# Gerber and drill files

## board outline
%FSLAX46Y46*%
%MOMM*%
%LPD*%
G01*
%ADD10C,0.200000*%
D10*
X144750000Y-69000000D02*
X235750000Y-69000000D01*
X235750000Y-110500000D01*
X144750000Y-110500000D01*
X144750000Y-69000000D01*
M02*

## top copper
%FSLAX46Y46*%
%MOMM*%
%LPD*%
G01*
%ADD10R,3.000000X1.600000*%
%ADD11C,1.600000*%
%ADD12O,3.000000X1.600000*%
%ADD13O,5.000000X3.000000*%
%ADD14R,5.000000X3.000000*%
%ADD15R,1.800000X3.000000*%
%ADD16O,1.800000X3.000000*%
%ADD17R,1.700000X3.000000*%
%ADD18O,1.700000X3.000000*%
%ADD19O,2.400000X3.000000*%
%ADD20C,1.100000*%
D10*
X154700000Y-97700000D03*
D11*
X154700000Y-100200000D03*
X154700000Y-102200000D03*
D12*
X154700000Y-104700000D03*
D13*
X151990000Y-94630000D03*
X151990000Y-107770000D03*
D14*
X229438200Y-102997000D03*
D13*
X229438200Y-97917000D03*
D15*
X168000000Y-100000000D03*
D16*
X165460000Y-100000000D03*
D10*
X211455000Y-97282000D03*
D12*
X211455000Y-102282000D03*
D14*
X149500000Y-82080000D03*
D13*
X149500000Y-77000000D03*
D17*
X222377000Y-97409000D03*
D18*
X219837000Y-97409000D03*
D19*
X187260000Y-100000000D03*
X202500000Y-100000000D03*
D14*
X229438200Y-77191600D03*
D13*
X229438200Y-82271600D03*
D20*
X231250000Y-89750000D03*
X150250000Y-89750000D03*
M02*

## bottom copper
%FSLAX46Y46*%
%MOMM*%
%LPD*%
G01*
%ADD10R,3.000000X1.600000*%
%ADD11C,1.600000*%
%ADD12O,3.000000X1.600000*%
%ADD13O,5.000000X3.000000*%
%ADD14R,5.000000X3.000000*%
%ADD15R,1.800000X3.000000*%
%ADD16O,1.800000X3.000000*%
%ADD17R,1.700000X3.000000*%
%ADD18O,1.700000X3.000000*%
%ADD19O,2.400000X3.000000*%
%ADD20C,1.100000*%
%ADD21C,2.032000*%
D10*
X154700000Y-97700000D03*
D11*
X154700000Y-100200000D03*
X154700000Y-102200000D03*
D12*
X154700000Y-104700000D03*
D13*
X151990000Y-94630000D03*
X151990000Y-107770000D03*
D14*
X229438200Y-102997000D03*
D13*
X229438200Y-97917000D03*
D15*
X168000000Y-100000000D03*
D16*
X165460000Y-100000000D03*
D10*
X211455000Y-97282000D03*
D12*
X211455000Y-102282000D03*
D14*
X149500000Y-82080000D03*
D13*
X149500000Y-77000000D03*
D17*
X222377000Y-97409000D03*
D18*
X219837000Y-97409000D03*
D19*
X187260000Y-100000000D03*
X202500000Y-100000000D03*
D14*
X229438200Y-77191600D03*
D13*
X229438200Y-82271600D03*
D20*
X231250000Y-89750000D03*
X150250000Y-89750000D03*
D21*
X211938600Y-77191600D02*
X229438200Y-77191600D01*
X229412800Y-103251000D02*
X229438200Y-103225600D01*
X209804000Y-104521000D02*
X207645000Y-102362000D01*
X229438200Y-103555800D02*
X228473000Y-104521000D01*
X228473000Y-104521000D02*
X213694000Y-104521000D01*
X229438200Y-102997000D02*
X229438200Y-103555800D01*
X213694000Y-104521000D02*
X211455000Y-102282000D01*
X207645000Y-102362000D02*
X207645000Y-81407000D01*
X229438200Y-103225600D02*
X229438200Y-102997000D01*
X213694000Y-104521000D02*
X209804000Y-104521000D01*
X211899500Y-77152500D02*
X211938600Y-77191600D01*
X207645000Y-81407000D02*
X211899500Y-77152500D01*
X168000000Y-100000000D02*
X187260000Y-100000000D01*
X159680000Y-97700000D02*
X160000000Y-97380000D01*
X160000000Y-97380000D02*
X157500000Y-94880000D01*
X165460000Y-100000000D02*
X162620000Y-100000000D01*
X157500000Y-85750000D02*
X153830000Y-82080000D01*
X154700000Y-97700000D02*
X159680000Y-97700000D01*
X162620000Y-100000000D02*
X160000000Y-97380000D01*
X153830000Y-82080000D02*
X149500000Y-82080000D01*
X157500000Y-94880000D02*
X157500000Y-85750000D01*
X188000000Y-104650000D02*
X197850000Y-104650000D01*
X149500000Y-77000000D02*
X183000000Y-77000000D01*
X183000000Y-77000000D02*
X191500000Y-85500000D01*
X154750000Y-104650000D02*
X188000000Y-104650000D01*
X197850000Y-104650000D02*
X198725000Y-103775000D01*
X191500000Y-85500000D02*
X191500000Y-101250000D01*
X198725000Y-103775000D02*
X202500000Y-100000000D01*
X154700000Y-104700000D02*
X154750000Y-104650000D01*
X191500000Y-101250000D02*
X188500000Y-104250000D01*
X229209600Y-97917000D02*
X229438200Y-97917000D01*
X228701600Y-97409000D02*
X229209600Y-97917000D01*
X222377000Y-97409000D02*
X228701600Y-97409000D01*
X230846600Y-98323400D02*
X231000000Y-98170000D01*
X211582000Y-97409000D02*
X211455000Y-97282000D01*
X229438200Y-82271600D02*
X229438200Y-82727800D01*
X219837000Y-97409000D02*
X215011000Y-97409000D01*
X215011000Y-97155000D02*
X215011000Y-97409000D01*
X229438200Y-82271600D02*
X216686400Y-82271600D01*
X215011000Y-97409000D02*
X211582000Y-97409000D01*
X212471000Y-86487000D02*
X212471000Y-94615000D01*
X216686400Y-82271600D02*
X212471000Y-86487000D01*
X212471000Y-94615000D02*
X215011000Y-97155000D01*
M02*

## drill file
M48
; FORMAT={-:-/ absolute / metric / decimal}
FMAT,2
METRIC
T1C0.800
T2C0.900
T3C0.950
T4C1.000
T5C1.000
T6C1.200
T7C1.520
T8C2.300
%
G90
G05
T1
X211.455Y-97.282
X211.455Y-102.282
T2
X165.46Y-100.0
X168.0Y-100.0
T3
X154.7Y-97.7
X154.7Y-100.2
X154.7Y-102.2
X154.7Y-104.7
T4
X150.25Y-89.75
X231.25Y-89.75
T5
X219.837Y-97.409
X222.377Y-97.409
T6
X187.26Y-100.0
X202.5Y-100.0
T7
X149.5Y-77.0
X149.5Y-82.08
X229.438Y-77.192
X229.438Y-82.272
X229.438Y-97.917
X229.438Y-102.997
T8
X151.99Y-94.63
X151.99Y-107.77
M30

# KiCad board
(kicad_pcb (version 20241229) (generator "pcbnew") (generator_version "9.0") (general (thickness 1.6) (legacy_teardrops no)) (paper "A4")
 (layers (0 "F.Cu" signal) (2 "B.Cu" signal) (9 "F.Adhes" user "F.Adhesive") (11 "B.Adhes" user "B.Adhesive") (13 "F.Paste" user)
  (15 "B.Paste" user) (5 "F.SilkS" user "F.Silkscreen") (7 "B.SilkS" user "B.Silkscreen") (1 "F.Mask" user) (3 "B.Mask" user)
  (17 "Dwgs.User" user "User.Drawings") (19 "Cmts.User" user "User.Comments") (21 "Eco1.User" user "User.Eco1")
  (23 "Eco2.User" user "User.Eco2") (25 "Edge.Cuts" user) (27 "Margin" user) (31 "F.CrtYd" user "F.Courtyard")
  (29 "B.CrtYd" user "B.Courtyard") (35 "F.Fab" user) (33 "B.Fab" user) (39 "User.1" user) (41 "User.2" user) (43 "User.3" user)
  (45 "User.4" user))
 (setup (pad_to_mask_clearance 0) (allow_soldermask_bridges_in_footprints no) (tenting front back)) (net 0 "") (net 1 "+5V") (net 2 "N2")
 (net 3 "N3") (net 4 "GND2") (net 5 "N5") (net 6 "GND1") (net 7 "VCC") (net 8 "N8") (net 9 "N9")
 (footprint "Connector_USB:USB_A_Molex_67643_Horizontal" (layer "F.Cu") (at 154.7 97.7 -90)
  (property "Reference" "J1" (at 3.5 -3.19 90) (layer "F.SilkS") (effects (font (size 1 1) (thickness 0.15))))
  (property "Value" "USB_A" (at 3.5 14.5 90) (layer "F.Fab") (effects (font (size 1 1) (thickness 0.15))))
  (pad "1" thru_hole rect (at 0 0 270) (size 1.6 3) (drill 0.95) (layers "*.Cu" "*.Mask") (remove_unused_layers no) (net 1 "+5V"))
  (pad "2" thru_hole circle (at 2.5 0 270) (size 1.6 1.6) (drill 0.95) (layers "*.Cu" "*.Mask") (remove_unused_layers no) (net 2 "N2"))
  (pad "3" thru_hole circle (at 4.5 0 270) (size 1.6 1.6) (drill 0.95) (layers "*.Cu" "*.Mask") (remove_unused_layers no) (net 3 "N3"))
  (pad "4" thru_hole oval (at 7 0 270) (size 1.6 3) (drill 0.95) (layers "*.Cu" "*.Mask") (remove_unused_layers no) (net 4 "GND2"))
  (pad "5" thru_hole oval (at -3.07 2.71 270) (size 3 5) (drill 2.3) (layers "*.Cu" "*.Mask") (remove_unused_layers no) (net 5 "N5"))
  (pad "5" thru_hole oval (at 10.07 2.71 270) (size 3 5) (drill 2.3) (layers "*.Cu" "*.Mask") (remove_unused_layers no) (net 5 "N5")))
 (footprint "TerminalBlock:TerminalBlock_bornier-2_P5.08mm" (layer "F.Cu") (at 229.4382 102.997 90)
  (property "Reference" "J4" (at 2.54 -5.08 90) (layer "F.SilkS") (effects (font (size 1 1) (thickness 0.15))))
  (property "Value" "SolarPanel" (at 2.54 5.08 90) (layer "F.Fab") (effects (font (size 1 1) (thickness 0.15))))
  (pad "1" thru_hole rect (at 0 0 90) (size 3 5) (drill 1.52) (layers "*.Cu" "*.Mask") (remove_unused_layers no) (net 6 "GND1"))
  (pad "2" thru_hole oval (at 5.08 0 90) (size 3 5) (drill 1.52) (layers "*.Cu" "*.Mask") (remove_unused_layers no) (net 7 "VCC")))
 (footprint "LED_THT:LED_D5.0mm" (layer "F.Cu") (at 168 100 180)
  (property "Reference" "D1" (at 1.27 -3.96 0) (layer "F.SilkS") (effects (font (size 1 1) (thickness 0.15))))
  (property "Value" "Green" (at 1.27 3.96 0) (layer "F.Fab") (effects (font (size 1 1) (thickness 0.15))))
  (pad "1" thru_hole rect (at 0 0 180) (size 1.8 3) (drill 0.9) (layers "*.Cu" "*.Mask") (remove_unused_layers no) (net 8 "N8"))
  (pad "2" thru_hole oval (at 2.54 0 180) (size 1.8 3) (drill 0.9) (layers "*.Cu" "*.Mask") (remove_unused_layers no) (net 1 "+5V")))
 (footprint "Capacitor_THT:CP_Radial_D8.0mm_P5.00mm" (layer "F.Cu") (at 211.455 97.282 -90)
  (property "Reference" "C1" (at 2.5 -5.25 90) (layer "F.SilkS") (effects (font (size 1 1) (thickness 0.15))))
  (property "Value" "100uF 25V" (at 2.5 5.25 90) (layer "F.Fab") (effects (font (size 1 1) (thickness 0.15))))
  (pad "1" thru_hole rect (at 0 0 270) (size 1.6 3) (drill 0.8) (layers "*.Cu" "*.Mask") (remove_unused_layers no) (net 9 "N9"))
  (pad "2" thru_hole oval (at 5 0 270) (size 1.6 3) (drill 0.8) (layers "*.Cu" "*.Mask") (remove_unused_layers no) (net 6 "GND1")))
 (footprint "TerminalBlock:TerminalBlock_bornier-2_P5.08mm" (layer "F.Cu") (at 149.5 82.08 90)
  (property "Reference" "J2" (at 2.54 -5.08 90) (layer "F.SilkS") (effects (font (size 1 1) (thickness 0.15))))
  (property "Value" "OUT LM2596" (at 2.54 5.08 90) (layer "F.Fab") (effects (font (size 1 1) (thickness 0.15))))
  (pad "1" thru_hole rect (at 0 0 90) (size 3 5) (drill 1.52) (layers "*.Cu" "*.Mask") (remove_unused_layers no) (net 1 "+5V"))
  (pad "2" thru_hole oval (at 5.08 0 90) (size 3 5) (drill 1.52) (layers "*.Cu" "*.Mask") (remove_unused_layers no) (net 4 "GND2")))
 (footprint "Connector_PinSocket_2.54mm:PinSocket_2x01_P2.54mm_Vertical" (layer "F.Cu") (at 222.377 97.409)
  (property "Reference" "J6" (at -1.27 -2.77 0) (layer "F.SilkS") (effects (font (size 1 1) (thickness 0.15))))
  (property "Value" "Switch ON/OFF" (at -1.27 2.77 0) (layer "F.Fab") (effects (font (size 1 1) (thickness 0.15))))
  (pad "1" thru_hole rect (at 0 0) (size 1.7 3) (drill 1) (layers "*.Cu" "*.Mask") (remove_unused_layers no) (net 7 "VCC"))
  (pad "2" thru_hole oval (at -2.54 0) (size 1.7 3) (drill 1) (layers "*.Cu" "*.Mask") (remove_unused_layers no) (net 9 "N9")))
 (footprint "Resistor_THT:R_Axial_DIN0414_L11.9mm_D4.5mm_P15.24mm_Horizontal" (layer "F.Cu") (at 187.26 100)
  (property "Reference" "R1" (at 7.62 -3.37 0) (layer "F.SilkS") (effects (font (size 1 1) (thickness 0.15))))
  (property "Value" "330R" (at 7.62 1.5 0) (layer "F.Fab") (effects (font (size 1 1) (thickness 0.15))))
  (pad "1" thru_hole oval (at 0 0) (size 2.4 3) (drill 1.2) (layers "*.Cu" "*.Mask") (remove_unused_layers no) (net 8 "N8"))
  (pad "2" thru_hole oval (at 15.24 0) (size 2.4 3) (drill 1.2) (layers "*.Cu" "*.Mask") (remove_unused_layers no) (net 4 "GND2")))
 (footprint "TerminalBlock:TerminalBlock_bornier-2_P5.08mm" (layer "F.Cu") (at 229.4382 77.1916 -90)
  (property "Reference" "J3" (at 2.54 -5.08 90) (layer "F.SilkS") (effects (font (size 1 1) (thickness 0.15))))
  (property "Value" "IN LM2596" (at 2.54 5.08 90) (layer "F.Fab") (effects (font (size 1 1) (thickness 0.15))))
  (pad "1" thru_hole rect (at 0 0 270) (size 3 5) (drill 1.52) (layers "*.Cu" "*.Mask") (remove_unused_layers no) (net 6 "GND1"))
  (pad "2" thru_hole oval (at 5.08 0 270) (size 3 5) (drill 1.52) (layers "*.Cu" "*.Mask") (remove_unused_layers no) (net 9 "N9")))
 (gr_rect (start 144.75 69) (end 235.75 110.5) (stroke (width 0.2) (type solid)) (fill no) (layer "Edge.Cuts"))
 (via (at 231.25 89.75) (size 1.1) (drill 1) (layers "F.Cu" "B.Cu") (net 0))
 (via (at 150.25 89.75) (size 1.1) (drill 1) (layers "F.Cu" "B.Cu") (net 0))
 (segment (start 211.9386 77.1916) (end 229.4382 77.1916) (width 2.032) (layer "B.Cu") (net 6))
 (segment (start 229.4128 103.251) (end 229.4382 103.2256) (width 2.032) (layer "B.Cu") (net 6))
 (segment (start 209.804 104.521) (end 207.645 102.362) (width 2.032) (layer "B.Cu") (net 6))
 (segment (start 229.4382 103.5558) (end 228.473 104.521) (width 2.032) (layer "B.Cu") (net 6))
 (segment (start 228.473 104.521) (end 213.694 104.521) (width 2.032) (layer "B.Cu") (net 6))
 (segment (start 229.4382 102.997) (end 229.4382 103.5558) (width 2.032) (layer "B.Cu") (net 6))
 (segment (start 213.694 104.521) (end 211.455 102.282) (width 2.032) (layer "B.Cu") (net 6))
 (segment (start 207.645 102.362) (end 207.645 81.407) (width 2.032) (layer "B.Cu") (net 6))
 (segment (start 229.4382 103.2256) (end 229.4382 102.997) (width 2.032) (layer "B.Cu") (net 6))
 (segment (start 213.694 104.521) (end 209.804 104.521) (width 2.032) (layer "B.Cu") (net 6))
 (segment (start 211.8995 77.1525) (end 211.9386 77.1916) (width 2.032) (layer "B.Cu") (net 6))
 (segment (start 207.645 81.407) (end 211.8995 77.1525) (width 2.032) (layer "B.Cu") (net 6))
 (segment (start 168 100) (end 187.26 100) (width 2.032) (layer "B.Cu") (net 8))
 (segment (start 159.68 97.7) (end 160 97.38) (width 2.032) (layer "B.Cu") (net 1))
 (segment (start 160 97.38) (end 157.5 94.88) (width 2.032) (layer "B.Cu") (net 1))
 (segment (start 165.46 100) (end 162.62 100) (width 2.032) (layer "B.Cu") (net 1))
 (segment (start 157.5 85.75) (end 153.83 82.08) (width 2.032) (layer "B.Cu") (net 1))
 (segment (start 154.7 97.7) (end 159.68 97.7) (width 2.032) (layer "B.Cu") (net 1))
 (segment (start 162.62 100) (end 160 97.38) (width 2.032) (layer "B.Cu") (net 1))
 (segment (start 153.83 82.08) (end 149.5 82.08) (width 2.032) (layer "B.Cu") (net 1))
 (segment (start 157.5 94.88) (end 157.5 85.75) (width 2.032) (layer "B.Cu") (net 1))
 (segment (start 188 104.65) (end 197.85 104.65) (width 2.032) (layer "B.Cu") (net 4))
 (segment (start 149.5 77) (end 183 77) (width 2.032) (layer "B.Cu") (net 4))
 (segment (start 183 77) (end 191.5 85.5) (width 2.032) (layer "B.Cu") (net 4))
 (segment (start 154.75 104.65) (end 188 104.65) (width 2.032) (layer "B.Cu") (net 4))
 (segment (start 197.85 104.65) (end 198.725 103.775) (width 2.032) (layer "B.Cu") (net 4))
 (segment (start 191.5 85.5) (end 191.5 101.25) (width 2.032) (layer "B.Cu") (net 4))
 (segment (start 198.725 103.775) (end 202.5 100) (width 2.032) (layer "B.Cu") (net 4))
 (segment (start 154.7 104.7) (end 154.75 104.65) (width 2.032) (layer "B.Cu") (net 4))
 (segment (start 191.5 101.25) (end 188.5 104.25) (width 2.032) (layer "B.Cu") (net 4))
 (segment (start 229.2096 97.917) (end 229.4382 97.917) (width 2.032) (layer "B.Cu") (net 7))
 (segment (start 228.7016 97.409) (end 229.2096 97.917) (width 2.032) (layer "B.Cu") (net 7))
 (segment (start 222.377 97.409) (end 228.7016 97.409) (width 2.032) (layer "B.Cu") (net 7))
 (segment (start 230.8466 98.3234) (end 231 98.17) (width 2.032) (layer "B.Cu") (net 7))
 (segment (start 211.582 97.409) (end 211.455 97.282) (width 2.032) (layer "B.Cu") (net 9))
 (segment (start 229.4382 82.2716) (end 229.4382 82.7278) (width 2.032) (layer "B.Cu") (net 9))
 (segment (start 219.837 97.409) (end 215.011 97.409) (width 2.032) (layer "B.Cu") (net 9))
 (segment (start 215.011 97.155) (end 215.011 97.409) (width 2.032) (layer "B.Cu") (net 9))
 (segment (start 229.4382 82.2716) (end 216.6864 82.2716) (width 2.032) (layer "B.Cu") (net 9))
 (segment (start 215.011 97.409) (end 211.582 97.409) (width 2.032) (layer "B.Cu") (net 9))
 (segment (start 212.471 86.487) (end 212.471 94.615) (width 2.032) (layer "B.Cu") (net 9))
 (segment (start 216.6864 82.2716) (end 212.471 86.487) (width 2.032) (layer "B.Cu") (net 9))
 (segment (start 212.471 94.615) (end 215.011 97.155) (width 2.032) (layer "B.Cu") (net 9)))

